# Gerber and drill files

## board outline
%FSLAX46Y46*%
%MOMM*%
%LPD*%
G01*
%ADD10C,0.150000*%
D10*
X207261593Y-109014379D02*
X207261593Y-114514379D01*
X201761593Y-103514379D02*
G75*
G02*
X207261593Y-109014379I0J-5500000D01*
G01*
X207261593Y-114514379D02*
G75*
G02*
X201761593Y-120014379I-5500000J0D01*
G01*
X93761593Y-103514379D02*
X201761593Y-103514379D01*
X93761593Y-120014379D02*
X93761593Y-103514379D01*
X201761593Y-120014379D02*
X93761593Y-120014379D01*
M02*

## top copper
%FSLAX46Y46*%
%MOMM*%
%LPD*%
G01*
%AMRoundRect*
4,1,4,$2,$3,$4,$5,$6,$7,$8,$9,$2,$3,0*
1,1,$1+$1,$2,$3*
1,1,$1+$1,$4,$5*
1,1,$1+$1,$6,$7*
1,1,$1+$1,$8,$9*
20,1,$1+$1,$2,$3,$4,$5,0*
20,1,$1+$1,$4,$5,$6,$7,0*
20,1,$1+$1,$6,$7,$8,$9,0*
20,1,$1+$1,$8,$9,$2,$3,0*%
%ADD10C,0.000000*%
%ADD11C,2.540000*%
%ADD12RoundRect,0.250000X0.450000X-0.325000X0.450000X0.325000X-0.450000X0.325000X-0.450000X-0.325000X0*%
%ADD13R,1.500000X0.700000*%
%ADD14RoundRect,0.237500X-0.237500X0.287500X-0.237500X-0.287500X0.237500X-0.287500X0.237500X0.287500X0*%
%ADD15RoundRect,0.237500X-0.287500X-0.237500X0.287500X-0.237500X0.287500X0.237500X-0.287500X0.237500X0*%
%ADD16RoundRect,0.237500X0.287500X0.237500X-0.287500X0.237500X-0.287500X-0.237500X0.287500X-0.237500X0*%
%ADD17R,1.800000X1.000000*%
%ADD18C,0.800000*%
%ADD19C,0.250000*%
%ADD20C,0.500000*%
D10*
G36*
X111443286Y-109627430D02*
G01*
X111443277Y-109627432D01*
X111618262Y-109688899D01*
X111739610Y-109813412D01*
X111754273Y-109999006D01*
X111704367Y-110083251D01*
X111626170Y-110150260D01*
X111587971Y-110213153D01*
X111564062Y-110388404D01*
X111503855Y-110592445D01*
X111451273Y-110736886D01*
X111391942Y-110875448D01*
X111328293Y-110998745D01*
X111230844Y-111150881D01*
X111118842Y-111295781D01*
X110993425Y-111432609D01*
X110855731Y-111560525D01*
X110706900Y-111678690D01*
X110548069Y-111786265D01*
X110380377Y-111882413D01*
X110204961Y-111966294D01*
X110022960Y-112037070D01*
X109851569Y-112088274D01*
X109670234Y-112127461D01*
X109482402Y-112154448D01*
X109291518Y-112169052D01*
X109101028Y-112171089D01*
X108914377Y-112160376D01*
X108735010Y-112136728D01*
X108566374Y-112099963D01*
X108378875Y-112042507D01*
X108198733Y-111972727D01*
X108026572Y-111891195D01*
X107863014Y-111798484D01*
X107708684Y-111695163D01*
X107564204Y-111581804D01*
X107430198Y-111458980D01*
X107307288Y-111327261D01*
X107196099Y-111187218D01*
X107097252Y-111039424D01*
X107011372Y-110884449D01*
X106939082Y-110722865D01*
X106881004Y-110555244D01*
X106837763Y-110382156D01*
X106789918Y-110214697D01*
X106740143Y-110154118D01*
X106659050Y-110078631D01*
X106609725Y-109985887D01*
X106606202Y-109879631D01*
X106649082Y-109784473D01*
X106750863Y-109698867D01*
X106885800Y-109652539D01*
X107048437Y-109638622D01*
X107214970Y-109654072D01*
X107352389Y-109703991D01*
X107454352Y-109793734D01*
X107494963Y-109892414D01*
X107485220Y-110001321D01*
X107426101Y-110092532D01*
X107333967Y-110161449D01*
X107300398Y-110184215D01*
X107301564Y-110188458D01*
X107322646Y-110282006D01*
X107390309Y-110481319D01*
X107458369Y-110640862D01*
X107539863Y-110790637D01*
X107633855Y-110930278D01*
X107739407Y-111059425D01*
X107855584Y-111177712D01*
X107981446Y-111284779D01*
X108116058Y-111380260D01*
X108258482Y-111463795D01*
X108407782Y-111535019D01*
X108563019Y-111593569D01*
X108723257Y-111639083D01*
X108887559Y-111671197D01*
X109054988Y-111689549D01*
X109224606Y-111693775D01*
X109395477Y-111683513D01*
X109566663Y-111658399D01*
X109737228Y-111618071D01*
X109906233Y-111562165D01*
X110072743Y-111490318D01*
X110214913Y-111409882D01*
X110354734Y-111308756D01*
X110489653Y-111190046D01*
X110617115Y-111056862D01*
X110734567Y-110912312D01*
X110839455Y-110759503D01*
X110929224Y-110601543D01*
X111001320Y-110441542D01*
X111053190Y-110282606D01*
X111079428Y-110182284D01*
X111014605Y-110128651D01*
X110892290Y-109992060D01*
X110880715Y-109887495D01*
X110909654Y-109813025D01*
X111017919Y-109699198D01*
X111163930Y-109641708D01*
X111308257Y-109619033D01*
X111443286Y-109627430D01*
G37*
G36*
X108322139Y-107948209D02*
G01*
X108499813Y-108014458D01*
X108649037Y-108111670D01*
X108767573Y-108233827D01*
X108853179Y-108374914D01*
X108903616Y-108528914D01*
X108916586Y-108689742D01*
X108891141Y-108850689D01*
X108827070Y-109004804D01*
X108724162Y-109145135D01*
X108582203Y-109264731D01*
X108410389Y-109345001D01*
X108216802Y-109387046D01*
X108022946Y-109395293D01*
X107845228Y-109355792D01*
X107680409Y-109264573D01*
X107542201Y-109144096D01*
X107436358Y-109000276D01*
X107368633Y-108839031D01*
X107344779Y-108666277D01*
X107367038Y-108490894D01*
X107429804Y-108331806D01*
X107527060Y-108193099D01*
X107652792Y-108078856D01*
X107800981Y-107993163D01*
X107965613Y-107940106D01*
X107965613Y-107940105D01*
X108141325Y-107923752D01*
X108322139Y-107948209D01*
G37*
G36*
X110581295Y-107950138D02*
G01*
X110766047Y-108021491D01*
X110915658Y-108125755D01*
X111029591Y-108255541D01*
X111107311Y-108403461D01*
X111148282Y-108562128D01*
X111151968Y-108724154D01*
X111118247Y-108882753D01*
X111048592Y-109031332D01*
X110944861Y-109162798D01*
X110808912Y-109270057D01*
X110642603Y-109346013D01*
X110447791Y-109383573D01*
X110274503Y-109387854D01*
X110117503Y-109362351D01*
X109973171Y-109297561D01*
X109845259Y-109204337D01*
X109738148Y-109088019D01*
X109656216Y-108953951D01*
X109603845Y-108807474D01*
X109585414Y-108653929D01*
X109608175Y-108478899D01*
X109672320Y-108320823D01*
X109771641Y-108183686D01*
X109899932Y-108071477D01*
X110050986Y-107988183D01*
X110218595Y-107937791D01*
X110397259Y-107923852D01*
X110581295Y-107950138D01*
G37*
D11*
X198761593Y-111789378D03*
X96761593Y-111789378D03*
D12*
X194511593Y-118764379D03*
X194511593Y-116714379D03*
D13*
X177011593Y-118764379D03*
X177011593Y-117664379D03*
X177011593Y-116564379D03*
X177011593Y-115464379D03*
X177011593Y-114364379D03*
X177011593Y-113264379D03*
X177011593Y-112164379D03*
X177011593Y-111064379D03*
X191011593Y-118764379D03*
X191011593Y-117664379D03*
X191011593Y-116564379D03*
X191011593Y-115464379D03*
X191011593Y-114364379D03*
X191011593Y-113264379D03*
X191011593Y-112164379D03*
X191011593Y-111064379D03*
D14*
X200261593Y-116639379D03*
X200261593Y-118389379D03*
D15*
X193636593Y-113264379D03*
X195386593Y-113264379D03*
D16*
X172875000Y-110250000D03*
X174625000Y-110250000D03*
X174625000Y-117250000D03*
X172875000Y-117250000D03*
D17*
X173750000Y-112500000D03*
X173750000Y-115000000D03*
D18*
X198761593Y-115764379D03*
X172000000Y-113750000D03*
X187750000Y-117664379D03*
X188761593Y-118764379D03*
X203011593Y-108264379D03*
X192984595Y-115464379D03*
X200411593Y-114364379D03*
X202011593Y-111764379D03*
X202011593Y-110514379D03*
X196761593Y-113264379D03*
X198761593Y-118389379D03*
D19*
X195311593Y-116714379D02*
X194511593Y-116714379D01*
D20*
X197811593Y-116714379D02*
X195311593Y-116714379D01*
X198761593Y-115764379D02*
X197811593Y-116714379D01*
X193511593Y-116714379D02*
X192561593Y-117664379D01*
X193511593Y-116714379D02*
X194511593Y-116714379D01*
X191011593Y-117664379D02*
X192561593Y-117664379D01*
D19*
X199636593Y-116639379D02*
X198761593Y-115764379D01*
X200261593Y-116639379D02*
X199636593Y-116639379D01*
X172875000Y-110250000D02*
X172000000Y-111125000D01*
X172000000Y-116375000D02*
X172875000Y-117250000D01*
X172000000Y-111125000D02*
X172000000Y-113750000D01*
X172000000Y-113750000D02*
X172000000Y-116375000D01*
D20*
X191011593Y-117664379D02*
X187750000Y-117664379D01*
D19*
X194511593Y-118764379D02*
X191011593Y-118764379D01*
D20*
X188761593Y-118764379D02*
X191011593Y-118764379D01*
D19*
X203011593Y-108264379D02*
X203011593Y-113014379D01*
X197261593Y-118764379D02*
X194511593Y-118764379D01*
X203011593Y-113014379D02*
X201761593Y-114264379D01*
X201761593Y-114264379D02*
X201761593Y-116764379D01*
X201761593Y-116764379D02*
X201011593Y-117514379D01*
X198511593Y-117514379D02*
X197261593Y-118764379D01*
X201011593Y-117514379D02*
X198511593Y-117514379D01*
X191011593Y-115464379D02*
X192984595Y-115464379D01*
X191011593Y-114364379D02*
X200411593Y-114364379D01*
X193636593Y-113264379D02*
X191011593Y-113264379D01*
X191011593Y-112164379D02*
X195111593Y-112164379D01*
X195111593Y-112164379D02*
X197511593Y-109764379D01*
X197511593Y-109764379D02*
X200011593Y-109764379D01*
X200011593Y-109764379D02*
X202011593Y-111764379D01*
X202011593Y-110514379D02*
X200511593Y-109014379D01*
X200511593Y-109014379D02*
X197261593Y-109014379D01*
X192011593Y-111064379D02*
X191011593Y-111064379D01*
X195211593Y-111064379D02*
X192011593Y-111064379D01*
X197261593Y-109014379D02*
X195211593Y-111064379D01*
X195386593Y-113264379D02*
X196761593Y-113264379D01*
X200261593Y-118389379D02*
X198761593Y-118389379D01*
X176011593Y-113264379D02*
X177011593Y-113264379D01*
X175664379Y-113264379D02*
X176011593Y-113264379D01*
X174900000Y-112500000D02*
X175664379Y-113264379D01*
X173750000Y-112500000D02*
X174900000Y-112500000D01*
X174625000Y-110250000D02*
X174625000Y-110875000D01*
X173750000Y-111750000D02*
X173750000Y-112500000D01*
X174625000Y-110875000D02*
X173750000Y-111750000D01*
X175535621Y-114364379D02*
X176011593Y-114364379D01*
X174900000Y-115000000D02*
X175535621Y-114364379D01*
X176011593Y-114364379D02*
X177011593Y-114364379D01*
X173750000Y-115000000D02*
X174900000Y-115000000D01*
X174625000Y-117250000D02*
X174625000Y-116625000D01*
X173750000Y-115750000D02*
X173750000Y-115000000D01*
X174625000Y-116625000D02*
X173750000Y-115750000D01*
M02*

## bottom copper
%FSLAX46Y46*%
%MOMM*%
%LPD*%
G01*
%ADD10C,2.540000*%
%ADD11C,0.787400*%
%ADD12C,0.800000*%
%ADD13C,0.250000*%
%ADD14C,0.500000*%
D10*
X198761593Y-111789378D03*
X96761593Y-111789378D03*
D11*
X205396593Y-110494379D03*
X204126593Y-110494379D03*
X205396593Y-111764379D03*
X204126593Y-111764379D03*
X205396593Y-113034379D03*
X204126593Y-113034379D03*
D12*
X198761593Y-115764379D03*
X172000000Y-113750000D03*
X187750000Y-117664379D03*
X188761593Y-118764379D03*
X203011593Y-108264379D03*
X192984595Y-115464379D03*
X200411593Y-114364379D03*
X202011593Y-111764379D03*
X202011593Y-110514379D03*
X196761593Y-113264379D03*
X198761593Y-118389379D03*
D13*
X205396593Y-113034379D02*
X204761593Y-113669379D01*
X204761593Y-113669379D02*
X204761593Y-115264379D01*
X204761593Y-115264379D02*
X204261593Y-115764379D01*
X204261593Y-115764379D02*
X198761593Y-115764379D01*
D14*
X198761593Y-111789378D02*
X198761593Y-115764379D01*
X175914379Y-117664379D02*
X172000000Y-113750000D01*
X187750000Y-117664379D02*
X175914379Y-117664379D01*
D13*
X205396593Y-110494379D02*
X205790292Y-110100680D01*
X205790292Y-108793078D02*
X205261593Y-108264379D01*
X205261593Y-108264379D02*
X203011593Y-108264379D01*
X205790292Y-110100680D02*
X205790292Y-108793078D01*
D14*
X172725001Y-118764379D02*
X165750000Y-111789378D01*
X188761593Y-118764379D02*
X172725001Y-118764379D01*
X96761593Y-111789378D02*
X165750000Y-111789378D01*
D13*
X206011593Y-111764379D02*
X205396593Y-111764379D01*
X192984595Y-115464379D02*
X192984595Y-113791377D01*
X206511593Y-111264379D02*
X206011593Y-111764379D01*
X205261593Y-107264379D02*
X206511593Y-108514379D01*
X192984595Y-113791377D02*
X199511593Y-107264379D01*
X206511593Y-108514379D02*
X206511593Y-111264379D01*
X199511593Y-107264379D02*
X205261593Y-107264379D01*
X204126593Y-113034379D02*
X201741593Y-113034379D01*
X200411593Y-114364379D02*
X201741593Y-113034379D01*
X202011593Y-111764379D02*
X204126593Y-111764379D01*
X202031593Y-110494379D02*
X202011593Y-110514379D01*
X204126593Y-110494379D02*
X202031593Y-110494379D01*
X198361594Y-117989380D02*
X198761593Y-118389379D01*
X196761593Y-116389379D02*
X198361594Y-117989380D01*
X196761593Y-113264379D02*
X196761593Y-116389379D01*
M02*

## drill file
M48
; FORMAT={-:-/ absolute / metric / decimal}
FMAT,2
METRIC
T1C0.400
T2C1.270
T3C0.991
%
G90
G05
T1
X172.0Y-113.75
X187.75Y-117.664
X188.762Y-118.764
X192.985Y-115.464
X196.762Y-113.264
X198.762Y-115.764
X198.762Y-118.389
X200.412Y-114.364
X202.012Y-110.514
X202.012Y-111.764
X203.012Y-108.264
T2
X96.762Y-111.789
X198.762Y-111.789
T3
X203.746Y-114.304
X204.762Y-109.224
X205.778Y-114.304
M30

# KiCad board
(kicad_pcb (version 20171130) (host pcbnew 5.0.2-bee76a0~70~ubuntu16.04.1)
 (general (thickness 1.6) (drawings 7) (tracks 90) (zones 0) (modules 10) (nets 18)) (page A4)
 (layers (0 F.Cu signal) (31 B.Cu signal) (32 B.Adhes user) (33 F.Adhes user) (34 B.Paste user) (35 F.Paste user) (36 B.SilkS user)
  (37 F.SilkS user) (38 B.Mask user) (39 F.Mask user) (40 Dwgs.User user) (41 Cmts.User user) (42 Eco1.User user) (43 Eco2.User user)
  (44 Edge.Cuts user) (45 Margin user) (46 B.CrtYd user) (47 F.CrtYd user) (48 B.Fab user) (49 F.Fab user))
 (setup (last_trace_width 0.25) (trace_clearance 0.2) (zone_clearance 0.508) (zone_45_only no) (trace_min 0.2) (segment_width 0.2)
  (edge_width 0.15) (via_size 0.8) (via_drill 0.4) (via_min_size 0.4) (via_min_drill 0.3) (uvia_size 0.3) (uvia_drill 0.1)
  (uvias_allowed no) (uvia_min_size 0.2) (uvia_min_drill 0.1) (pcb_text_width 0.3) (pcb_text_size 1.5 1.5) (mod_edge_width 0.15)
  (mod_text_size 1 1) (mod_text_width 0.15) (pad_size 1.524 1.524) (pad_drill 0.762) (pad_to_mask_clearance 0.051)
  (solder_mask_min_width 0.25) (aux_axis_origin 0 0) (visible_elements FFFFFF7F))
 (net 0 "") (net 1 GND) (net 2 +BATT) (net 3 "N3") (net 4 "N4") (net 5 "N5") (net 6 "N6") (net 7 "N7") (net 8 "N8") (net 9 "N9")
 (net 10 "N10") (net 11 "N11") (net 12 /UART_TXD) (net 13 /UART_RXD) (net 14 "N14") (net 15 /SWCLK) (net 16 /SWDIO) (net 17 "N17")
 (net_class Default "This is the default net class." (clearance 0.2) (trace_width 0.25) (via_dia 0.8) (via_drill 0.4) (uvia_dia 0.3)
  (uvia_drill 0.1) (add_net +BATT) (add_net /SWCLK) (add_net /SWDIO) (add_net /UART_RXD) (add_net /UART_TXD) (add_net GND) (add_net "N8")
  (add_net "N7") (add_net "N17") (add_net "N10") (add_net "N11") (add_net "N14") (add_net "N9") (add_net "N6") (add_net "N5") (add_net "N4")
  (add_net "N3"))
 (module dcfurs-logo (layer F.Cu) (at 109.25 111.75)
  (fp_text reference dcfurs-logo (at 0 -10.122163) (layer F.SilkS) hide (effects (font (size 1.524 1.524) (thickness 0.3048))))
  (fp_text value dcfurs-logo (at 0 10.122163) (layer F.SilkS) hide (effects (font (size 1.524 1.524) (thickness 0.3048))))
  (fp_poly
   (pts (xy 0.968595 -3.812209) (xy -0.482427 -3.516173) (xy -0.600963 -3.63833) (xy -0.750187 -3.735542) (xy -0.927861 -3.801791)
    (xy -1.108675 -3.826248) (xy -1.284387 -3.809895) (xy -1.284387 -3.809894) (xy -1.449019 -3.756837) (xy -1.597208 -3.671144)
    (xy -1.72294 -3.556901) (xy -1.820196 -3.418194) (xy -1.882962 -3.259106) (xy -1.905221 -3.083723) (xy -1.881367 -2.910969)
    (xy -1.813642 -2.749724) (xy -1.707799 -2.605904) (xy -1.569591 -2.485427) (xy -1.404772 -2.394208) (xy -1.227054 -2.354707)
    (xy -1.033198 -2.362954) (xy -0.839611 -2.404999) (xy -0.667797 -2.485269) (xy -0.525838 -2.604865) (xy -0.42293 -2.745196)
    (xy -0.358859 -2.899311) (xy -0.333414 -3.060258) (xy -0.346384 -3.221086) (xy -0.396821 -3.375086) (xy -0.482427 -3.516173)
    (xy 0.968595 -3.812209) (xy 0.800986 -3.761817) (xy 0.649932 -3.678523) (xy 0.521641 -3.566314) (xy -1.616145 -0.819722)
    (xy -1.710137 -0.959363) (xy -1.791631 -1.109138) (xy -1.859691 -1.268681) (xy -1.927354 -1.467994) (xy -1.948436 -1.561542)
    (xy -1.949602 -1.565785) (xy -1.916033 -1.588551) (xy -1.823899 -1.657468) (xy -1.76478 -1.748679) (xy -1.755037 -1.857586)
    (xy -1.795648 -1.956266) (xy -1.897611 -2.046009) (xy -2.03503 -2.095928) (xy -2.201563 -2.111378) (xy -2.3642 -2.097461)
    (xy -2.499137 -2.051133) (xy -2.600918 -1.965527) (xy -2.643798 -1.870369) (xy -2.640275 -1.764113) (xy -2.59095 -1.671369)
    (xy -2.509857 -1.595882) (xy -2.460082 -1.535303) (xy -2.412237 -1.367844) (xy -2.368996 -1.194756) (xy -2.310918 -1.027135)
    (xy -2.238628 -0.865551) (xy -2.152748 -0.710576) (xy -2.053901 -0.562782) (xy -1.942712 -0.422739) (xy -1.819802 -0.29102)
    (xy -1.685796 -0.168196) (xy -1.541316 -0.054837) (xy -1.386986 0.048484) (xy -1.223428 0.141195) (xy -1.051267 0.222727)
    (xy -0.871125 0.292507) (xy -0.683626 0.349963) (xy -0.51499 0.386728) (xy -0.335623 0.410376) (xy -0.148972 0.421089)
    (xy 0.041518 0.419052) (xy 0.232402 0.404448) (xy 0.420234 0.377461) (xy 0.601569 0.338274) (xy 0.77296 0.28707) (xy 0.954961 0.216294)
    (xy 1.130377 0.132413) (xy 1.298069 0.036265) (xy 1.4569 -0.07131) (xy 1.605731 -0.189475) (xy 1.743425 -0.317391)
    (xy 1.868842 -0.454219) (xy 1.980844 -0.599119) (xy 2.078293 -0.751255) (xy 2.141942 -0.874552) (xy 2.201273 -1.013114)
    (xy 2.253855 -1.157555) (xy 2.314062 -1.361596) (xy 2.337971 -1.536847) (xy 2.37617 -1.59974) (xy 2.454367 -1.666749)
    (xy 2.504273 -1.750994) (xy 2.48961 -1.936588) (xy 2.368262 -2.061101) (xy 2.193277 -2.122568) (xy 2.193286 -2.12257)
    (xy 2.058257 -2.130967) (xy 1.91393 -2.108292) (xy 1.767919 -2.050802) (xy 1.659654 -1.936975) (xy 1.630715 -1.862505)
    (xy 1.64229 -1.75794) (xy 1.764605 -1.621349) (xy 1.829428 -1.567716) (xy 1.80319 -1.467394) (xy 1.75132 -1.308458)
    (xy 1.679224 -1.148457) (xy 1.589455 -0.990497) (xy 1.484567 -0.837688) (xy 1.367115 -0.693138) (xy 1.239653 -0.559954)
    (xy 1.104734 -0.441244) (xy 0.964913 -0.340118) (xy 0.822743 -0.259682) (xy 0.656233 -0.187835) (xy 0.487228 -0.131929)
    (xy 0.316663 -0.091601) (xy 0.145477 -0.066487) (xy -0.025394 -0.056225) (xy -0.195012 -0.060451) (xy -0.362441 -0.078803)
    (xy -0.526743 -0.110917) (xy -0.686981 -0.156431) (xy -0.842218 -0.214981) (xy -0.991518 -0.286205) (xy -1.133942 -0.36974)
    (xy -1.268554 -0.465221) (xy -1.394416 -0.572288) (xy -1.510593 -0.690575) (xy -1.616145 -0.819722) (xy 0.521641 -3.566314)
    (xy 0.42232 -3.429177) (xy 0.358175 -3.271101) (xy 0.335414 -3.096071) (xy 0.353845 -2.942526) (xy 0.406216 -2.796049)
    (xy 0.488148 -2.661981) (xy 0.595259 -2.545663) (xy 0.723171 -2.452439) (xy 0.867503 -2.387649) (xy 1.024503 -2.362146)
    (xy 1.197791 -2.366427) (xy 1.392603 -2.403987) (xy 1.558912 -2.479943) (xy 1.694861 -2.587202) (xy 1.798592 -2.718668)
    (xy 1.868247 -2.867247) (xy 1.901968 -3.025846) (xy 1.898282 -3.187872) (xy 1.857311 -3.346539) (xy 1.779591 -3.494459)
    (xy 1.665658 -3.624245) (xy 1.516047 -3.728509) (xy 1.331295 -3.799862) (xy 1.147259 -3.826148) (xy 0.968595 -3.812209))
   (layer F.Cu) (width 0)))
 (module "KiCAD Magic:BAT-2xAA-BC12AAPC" (layer B.Cu) (at 147.761593 111.789378 180)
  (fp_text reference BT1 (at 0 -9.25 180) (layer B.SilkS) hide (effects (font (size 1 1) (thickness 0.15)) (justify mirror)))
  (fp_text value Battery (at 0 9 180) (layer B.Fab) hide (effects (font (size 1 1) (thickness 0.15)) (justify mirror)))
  (pad 2 thru_hole circle (at -51 0 180) (size 2.54 2.54) (drill 1.27) (layers *.Cu *.Mask) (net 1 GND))
  (pad 1 thru_hole circle (at 51 0 180) (size 2.54 2.54) (drill 1.27) (layers *.Cu *.Mask) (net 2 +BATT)))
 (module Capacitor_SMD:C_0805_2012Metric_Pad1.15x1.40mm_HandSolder (layer F.Cu) (at 194.511593 117.739379 90)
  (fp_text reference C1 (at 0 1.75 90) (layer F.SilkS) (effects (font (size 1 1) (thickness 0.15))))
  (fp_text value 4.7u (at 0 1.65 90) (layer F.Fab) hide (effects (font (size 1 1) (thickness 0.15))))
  (pad 1 smd roundrect (at -1.025 0 90) (size 1.15 1.4) (layers F.Cu F.Paste F.Mask) (roundrect_rratio 0.217391) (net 2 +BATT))
  (pad 2 smd roundrect (at 1.025 0 90) (size 1.15 1.4) (layers F.Cu F.Paste F.Mask) (roundrect_rratio 0.217391) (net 1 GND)))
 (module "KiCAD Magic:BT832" (layer F.Cu) (at 184.011593 111.764379)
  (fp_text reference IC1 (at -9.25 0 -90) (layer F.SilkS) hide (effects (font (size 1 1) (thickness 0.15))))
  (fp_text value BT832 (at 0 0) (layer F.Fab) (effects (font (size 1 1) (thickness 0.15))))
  (pad 8 smd rect (at -7 7) (size 1.5 0.7) (layers F.Cu F.Paste F.Mask) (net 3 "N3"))
  (pad 7 smd rect (at -7 5.9) (size 1.5 0.7) (layers F.Cu F.Paste F.Mask) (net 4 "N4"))
  (pad 6 smd rect (at -7 4.8) (size 1.5 0.7) (layers F.Cu F.Paste F.Mask) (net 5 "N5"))
  (pad 5 smd rect (at -7 3.7) (size 1.5 0.7) (layers F.Cu F.Paste F.Mask) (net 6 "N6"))
  (pad 4 smd rect (at -7 2.6) (size 1.5 0.7) (layers F.Cu F.Paste F.Mask) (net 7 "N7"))
  (pad 3 smd rect (at -7 1.5) (size 1.5 0.7) (layers F.Cu F.Paste F.Mask) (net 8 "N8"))
  (pad 2 smd rect (at -7 0.4) (size 1.5 0.7) (layers F.Cu F.Paste F.Mask) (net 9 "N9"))
  (pad 1 smd rect (at -7 -0.7) (size 1.5 0.7) (layers F.Cu F.Paste F.Mask) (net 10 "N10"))
  (pad 9 smd rect (at 7 7) (size 1.5 0.7) (layers F.Cu F.Paste F.Mask) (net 2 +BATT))
  (pad 10 smd rect (at 7 5.9) (size 1.5 0.7) (layers F.Cu F.Paste F.Mask) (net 1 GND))
  (pad 11 smd rect (at 7 4.8) (size 1.5 0.7) (layers F.Cu F.Paste F.Mask) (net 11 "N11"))
  (pad 12 smd rect (at 7 3.7) (size 1.5 0.7) (layers F.Cu F.Paste F.Mask) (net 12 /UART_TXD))
  (pad 13 smd rect (at 7 2.6) (size 1.5 0.7) (layers F.Cu F.Paste F.Mask) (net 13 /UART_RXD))
  (pad 14 smd rect (at 7 1.5) (size 1.5 0.7) (layers F.Cu F.Paste F.Mask) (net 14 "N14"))
  (pad 15 smd rect (at 7 0.4) (size 1.5 0.7) (layers F.Cu F.Paste F.Mask) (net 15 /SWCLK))
  (pad 16 smd rect (at 7 -0.7) (size 1.5 0.7) (layers F.Cu F.Paste F.Mask) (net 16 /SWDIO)))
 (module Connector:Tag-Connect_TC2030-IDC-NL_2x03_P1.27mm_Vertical (layer B.Cu) (at 204.761593 111.764379 270)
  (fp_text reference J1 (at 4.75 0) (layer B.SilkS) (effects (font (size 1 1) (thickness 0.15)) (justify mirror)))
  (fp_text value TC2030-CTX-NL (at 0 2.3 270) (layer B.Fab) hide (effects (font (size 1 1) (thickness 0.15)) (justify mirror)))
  (pad "" np_thru_hole circle (at 2.54 1.016 270) (size 0.9906 0.9906) (drill 0.9906) (layers *.Cu *.Mask))
  (pad "" np_thru_hole circle (at 2.54 -1.016 270) (size 0.9906 0.9906) (drill 0.9906) (layers *.Cu *.Mask))
  (pad "" np_thru_hole circle (at -2.54 0 270) (size 0.9906 0.9906) (drill 0.9906) (layers *.Cu *.Mask))
  (pad 1 connect circle (at -1.27 -0.635 270) (size 0.7874 0.7874) (layers B.Cu B.Mask) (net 2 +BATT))
  (pad 2 connect circle (at -1.27 0.635 270) (size 0.7874 0.7874) (layers B.Cu B.Mask) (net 16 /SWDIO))
  (pad 3 connect circle (at 0 -0.635 270) (size 0.7874 0.7874) (layers B.Cu B.Mask) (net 12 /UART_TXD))
  (pad 4 connect circle (at 0 0.635 270) (size 0.7874 0.7874) (layers B.Cu B.Mask) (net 15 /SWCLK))
  (pad 5 connect circle (at 1.27 -0.635 270) (size 0.7874 0.7874) (layers B.Cu B.Mask) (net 1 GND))
  (pad 6 connect circle (at 1.27 0.635 270) (size 0.7874 0.7874) (layers B.Cu B.Mask) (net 13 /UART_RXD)))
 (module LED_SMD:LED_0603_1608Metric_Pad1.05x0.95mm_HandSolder (layer F.Cu) (at 200.261593 117.514379 270)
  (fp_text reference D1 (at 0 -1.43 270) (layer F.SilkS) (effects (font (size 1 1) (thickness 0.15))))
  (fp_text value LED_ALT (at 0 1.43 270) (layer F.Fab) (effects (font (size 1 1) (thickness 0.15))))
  (pad 1 smd roundrect (at -0.875 0 270) (size 1.05 0.95) (layers F.Cu F.Paste F.Mask) (roundrect_rratio 0.25) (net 1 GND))
  (pad 2 smd roundrect (at 0.875 0 270) (size 1.05 0.95) (layers F.Cu F.Paste F.Mask) (roundrect_rratio 0.25) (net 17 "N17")))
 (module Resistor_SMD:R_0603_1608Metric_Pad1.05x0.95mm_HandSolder (layer F.Cu) (at 194.511593 113.264379)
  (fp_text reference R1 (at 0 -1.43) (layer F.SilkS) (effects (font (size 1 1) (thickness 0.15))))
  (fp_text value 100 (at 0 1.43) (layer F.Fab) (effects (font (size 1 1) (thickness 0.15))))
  (pad 1 smd roundrect (at -0.875 0) (size 1.05 0.95) (layers F.Cu F.Paste F.Mask) (roundrect_rratio 0.25) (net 14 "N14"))
  (pad 2 smd roundrect (at 0.875 0) (size 1.05 0.95) (layers F.Cu F.Paste F.Mask) (roundrect_rratio 0.25) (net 17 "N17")))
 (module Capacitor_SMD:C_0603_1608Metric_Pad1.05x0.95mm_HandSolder (layer F.Cu) (at 173.75 110.25 180)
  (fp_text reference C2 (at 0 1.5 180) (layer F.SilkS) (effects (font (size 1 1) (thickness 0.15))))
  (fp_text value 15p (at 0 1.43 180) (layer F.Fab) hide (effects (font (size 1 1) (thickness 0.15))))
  (pad 2 smd roundrect (at 0.875 0 180) (size 1.05 0.95) (layers F.Cu F.Paste F.Mask) (roundrect_rratio 0.25) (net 1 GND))
  (pad 1 smd roundrect (at -0.875 0 180) (size 1.05 0.95) (layers F.Cu F.Paste F.Mask) (roundrect_rratio 0.25) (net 8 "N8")))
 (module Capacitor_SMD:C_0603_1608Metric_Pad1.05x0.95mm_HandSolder (layer F.Cu) (at 173.75 117.25 180)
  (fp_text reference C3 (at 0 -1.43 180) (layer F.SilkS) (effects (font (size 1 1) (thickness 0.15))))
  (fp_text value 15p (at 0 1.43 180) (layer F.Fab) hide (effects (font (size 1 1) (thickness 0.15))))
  (pad 1 smd roundrect (at -0.875 0 180) (size 1.05 0.95) (layers F.Cu F.Paste F.Mask) (roundrect_rratio 0.25) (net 7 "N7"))
  (pad 2 smd roundrect (at 0.875 0 180) (size 1.05 0.95) (layers F.Cu F.Paste F.Mask) (roundrect_rratio 0.25) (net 1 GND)))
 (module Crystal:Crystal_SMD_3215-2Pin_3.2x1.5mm (layer F.Cu) (at 173.75 113.75 90)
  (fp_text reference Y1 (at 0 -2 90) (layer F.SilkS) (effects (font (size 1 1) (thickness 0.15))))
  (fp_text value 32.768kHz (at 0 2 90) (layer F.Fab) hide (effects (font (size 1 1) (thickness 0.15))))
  (pad 1 smd rect (at 1.25 0 90) (size 1 1.8) (layers F.Cu F.Paste F.Mask) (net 8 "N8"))
  (pad 2 smd rect (at -1.25 0 90) (size 1 1.8) (layers F.Cu F.Paste F.Mask) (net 7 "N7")))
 (gr_line (start 207.261593 109.014379) (end 207.261593 114.514379) (layer Edge.Cuts) (width 0.15))
 (gr_arc (start 201.761593 109.014379) (end 207.261593 109.014379) (angle -90) (layer Edge.Cuts) (width 0.15))
 (gr_arc (start 201.761593 114.514379) (end 201.761593 120.014379) (angle -90) (layer Edge.Cuts) (width 0.15))
 (gr_line (start 93.761593 103.514379) (end 201.761593 103.514379) (layer Edge.Cuts) (width 0.15))
 (gr_line (start 93.761593 120.014379) (end 93.761593 103.514379) (layer Edge.Cuts) (width 0.15))
 (gr_line (start 201.761593 120.014379) (end 93.761593 120.014379) (layer Edge.Cuts) (width 0.15))
 (segment (start 195.311593 116.714379) (end 194.511593 116.714379) (width 0.25) (layer F.Cu) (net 1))
 (segment (start 197.811593 116.714379) (end 195.311593 116.714379) (width 0.5) (layer F.Cu) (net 1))
 (segment (start 198.761593 115.764379) (end 197.811593 116.714379) (width 0.5) (layer F.Cu) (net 1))
 (segment (start 205.396593 113.034379) (end 204.761593 113.669379) (width 0.25) (layer B.Cu) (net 1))
 (segment (start 204.761593 113.669379) (end 204.761593 115.264379) (width 0.25) (layer B.Cu) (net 1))
 (segment (start 204.761593 115.264379) (end 204.261593 115.764379) (width 0.25) (layer B.Cu) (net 1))
 (via (at 198.761593 115.764379) (size 0.8) (drill 0.4) (layers F.Cu B.Cu) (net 1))
 (segment (start 204.261593 115.764379) (end 198.761593 115.764379) (width 0.25) (layer B.Cu) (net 1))
 (segment (start 193.511593 116.714379) (end 192.561593 117.664379) (width 0.5) (layer F.Cu) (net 1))
 (segment (start 193.511593 116.714379) (end 194.511593 116.714379) (width 0.5) (layer F.Cu) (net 1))
 (segment (start 198.761593 111.789378) (end 198.761593 115.764379) (width 0.5) (layer B.Cu) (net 1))
 (segment (start 191.011593 117.664379) (end 192.561593 117.664379) (width 0.5) (layer F.Cu) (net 1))
 (segment (start 199.636593 116.639379) (end 198.761593 115.764379) (width 0.25) (layer F.Cu) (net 1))
 (segment (start 200.261593 116.639379) (end 199.636593 116.639379) (width 0.25) (layer F.Cu) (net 1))
 (segment (start 172.875 110.25) (end 172 111.125) (width 0.25) (layer F.Cu) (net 1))
 (segment (start 172 116.375) (end 172.875 117.25) (width 0.25) (layer F.Cu) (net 1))
 (segment (start 172 111.125) (end 172 113.75) (width 0.25) (layer F.Cu) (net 1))
 (via (at 172 113.75) (size 0.8) (drill 0.4) (layers F.Cu B.Cu) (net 1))
 (segment (start 172 113.75) (end 172 116.375) (width 0.25) (layer F.Cu) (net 1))
 (segment (start 191.011593 117.664379) (end 187.75 117.664379) (width 0.5) (layer F.Cu) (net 1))
 (via (at 187.75 117.664379) (size 0.8) (drill 0.4) (layers F.Cu B.Cu) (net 1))
 (segment (start 175.914379 117.664379) (end 172 113.75) (width 0.5) (layer B.Cu) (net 1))
 (segment (start 187.75 117.664379) (end 175.914379 117.664379) (width 0.5) (layer B.Cu) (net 1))
 (segment (start 194.511593 118.764379) (end 191.011593 118.764379) (width 0.25) (layer F.Cu) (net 2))
 (via (at 188.761593 118.764379) (size 0.8) (drill 0.4) (layers F.Cu B.Cu) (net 2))
 (segment (start 188.761593 118.764379) (end 191.011593 118.764379) (width 0.5) (layer F.Cu) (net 2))
 (segment (start 205.396593 110.494379) (end 205.790292 110.10068) (width 0.25) (layer B.Cu) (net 2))
 (segment (start 205.790292 108.793078) (end 205.261593 108.264379) (width 0.25) (layer B.Cu) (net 2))
 (via (at 203.011593 108.264379) (size 0.8) (drill 0.4) (layers F.Cu B.Cu) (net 2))
 (segment (start 205.261593 108.264379) (end 203.011593 108.264379) (width 0.25) (layer B.Cu) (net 2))
 (segment (start 203.011593 108.264379) (end 203.011593 113.014379) (width 0.25) (layer F.Cu) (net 2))
 (segment (start 197.261593 118.764379) (end 194.511593 118.764379) (width 0.25) (layer F.Cu) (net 2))
 (segment (start 205.790292 110.10068) (end 205.790292 108.793078) (width 0.25) (layer B.Cu) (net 2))
 (segment (start 203.011593 113.014379) (end 201.761593 114.264379) (width 0.25) (layer F.Cu) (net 2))
 (segment (start 201.761593 114.264379) (end 201.761593 116.764379) (width 0.25) (layer F.Cu) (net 2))
 (segment (start 201.761593 116.764379) (end 201.011593 117.514379) (width 0.25) (layer F.Cu) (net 2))
 (segment (start 198.511593 117.514379) (end 197.261593 118.764379) (width 0.25) (layer F.Cu) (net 2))
 (segment (start 201.011593 117.514379) (end 198.511593 117.514379) (width 0.25) (layer F.Cu) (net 2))
 (segment (start 172.725001 118.764379) (end 165.75 111.789378) (width 0.5) (layer B.Cu) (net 2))
 (segment (start 188.761593 118.764379) (end 172.725001 118.764379) (width 0.5) (layer B.Cu) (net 2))
 (segment (start 96.761593 111.789378) (end 165.75 111.789378) (width 0.5) (layer B.Cu) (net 2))
 (segment (start 191.011593 115.464379) (end 192.984595 115.464379) (width 0.25) (layer F.Cu) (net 12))
 (via (at 192.984595 115.464379) (size 0.8) (drill 0.4) (layers F.Cu B.Cu) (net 12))
 (segment (start 206.011593 111.764379) (end 205.396593 111.764379) (width 0.25) (layer B.Cu) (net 12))
 (segment (start 192.984595 115.464379) (end 192.984595 113.791377) (width 0.25) (layer B.Cu) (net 12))
 (segment (start 206.511593 111.264379) (end 206.011593 111.764379) (width 0.25) (layer B.Cu) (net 12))
 (segment (start 205.261593 107.264379) (end 206.511593 108.514379) (width 0.25) (layer B.Cu) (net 12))
 (segment (start 192.984595 113.791377) (end 199.511593 107.264379) (width 0.25) (layer B.Cu) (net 12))
 (segment (start 206.511593 108.514379) (end 206.511593 111.264379) (width 0.25) (layer B.Cu) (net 12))
 (segment (start 199.511593 107.264379) (end 205.261593 107.264379) (width 0.25) (layer B.Cu) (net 12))
 (via (at 200.411593 114.364379) (size 0.8) (drill 0.4) (layers F.Cu B.Cu) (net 13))
 (segment (start 204.126593 113.034379) (end 201.741593 113.034379) (width 0.25) (layer B.Cu) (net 13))
 (segment (start 200.411593 114.364379) (end 201.741593 113.034379) (width 0.25) (layer B.Cu) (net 13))
 (segment (start 191.011593 114.364379) (end 200.411593 114.364379) (width 0.25) (layer F.Cu) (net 13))
 (segment (start 193.636593 113.264379) (end 191.011593 113.264379) (width 0.25) (layer F.Cu) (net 14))
 (segment (start 191.011593 112.164379) (end 195.111593 112.164379) (width 0.25) (layer F.Cu) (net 15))
 (segment (start 195.111593 112.164379) (end 197.511593 109.764379) (width 0.25) (layer F.Cu) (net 15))
 (segment (start 197.511593 109.764379) (end 200.011593 109.764379) (width 0.25) (layer F.Cu) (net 15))
 (via (at 202.011593 111.764379) (size 0.8) (drill 0.4) (layers F.Cu B.Cu) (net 15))
 (segment (start 200.011593 109.764379) (end 202.011593 111.764379) (width 0.25) (layer F.Cu) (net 15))
 (segment (start 202.011593 111.764379) (end 204.126593 111.764379) (width 0.25) (layer B.Cu) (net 15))
 (via (at 202.011593 110.514379) (size 0.8) (drill 0.4) (layers F.Cu B.Cu) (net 16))
 (segment (start 202.031593 110.494379) (end 202.011593 110.514379) (width 0.25) (layer B.Cu) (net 16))
 (segment (start 204.126593 110.494379) (end 202.031593 110.494379) (width 0.25) (layer B.Cu) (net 16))
 (segment (start 202.011593 110.514379) (end 200.511593 109.014379) (width 0.25) (layer F.Cu) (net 16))
 (segment (start 200.511593 109.014379) (end 197.261593 109.014379) (width 0.25) (layer F.Cu) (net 16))
 (segment (start 192.011593 111.064379) (end 191.011593 111.064379) (width 0.25) (layer F.Cu) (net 16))
 (segment (start 195.211593 111.064379) (end 192.011593 111.064379) (width 0.25) (layer F.Cu) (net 16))
 (segment (start 197.261593 109.014379) (end 195.211593 111.064379) (width 0.25) (layer F.Cu) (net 16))
 (via (at 196.761593 113.264379) (size 0.8) (drill 0.4) (layers F.Cu B.Cu) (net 17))
 (segment (start 195.386593 113.264379) (end 196.761593 113.264379) (width 0.25) (layer F.Cu) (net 17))
 (via (at 198.761593 118.389379) (size 0.8) (drill 0.4) (layers F.Cu B.Cu) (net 17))
 (segment (start 198.361594 117.98938) (end 198.761593 118.389379) (width 0.25) (layer B.Cu) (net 17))
 (segment (start 196.761593 116.389379) (end 198.361594 117.98938) (width 0.25) (layer B.Cu) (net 17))
 (segment (start 196.761593 113.264379) (end 196.761593 116.389379) (width 0.25) (layer B.Cu) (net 17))
 (segment (start 200.261593 118.389379) (end 198.761593 118.389379) (width 0.25) (layer F.Cu) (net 17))
 (segment (start 176.011593 113.264379) (end 177.011593 113.264379) (width 0.25) (layer F.Cu) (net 8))
 (segment (start 175.664379 113.264379) (end 176.011593 113.264379) (width 0.25) (layer F.Cu) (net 8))
 (segment (start 174.9 112.5) (end 175.664379 113.264379) (width 0.25) (layer F.Cu) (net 8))
 (segment (start 173.75 112.5) (end 174.9 112.5) (width 0.25) (layer F.Cu) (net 8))
 (segment (start 174.625 110.25) (end 174.625 110.875) (width 0.25) (layer F.Cu) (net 8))
 (segment (start 173.75 111.75) (end 173.75 112.5) (width 0.25) (layer F.Cu) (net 8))
 (segment (start 174.625 110.875) (end 173.75 111.75) (width 0.25) (layer F.Cu) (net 8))
 (segment (start 175.535621 114.364379) (end 176.011593 114.364379) (width 0.25) (layer F.Cu) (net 7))
 (segment (start 174.9 115) (end 175.535621 114.364379) (width 0.25) (layer F.Cu) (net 7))
 (segment (start 176.011593 114.364379) (end 177.011593 114.364379) (width 0.25) (layer F.Cu) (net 7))
 (segment (start 173.75 115) (end 174.9 115) (width 0.25) (layer F.Cu) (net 7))
 (segment (start 174.625 117.25) (end 174.625 116.625) (width 0.25) (layer F.Cu) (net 7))
 (segment (start 173.75 115.75) (end 173.75 115) (width 0.25) (layer F.Cu) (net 7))
 (segment (start 174.625 116.625) (end 173.75 115.75) (width 0.25) (layer F.Cu) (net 7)))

